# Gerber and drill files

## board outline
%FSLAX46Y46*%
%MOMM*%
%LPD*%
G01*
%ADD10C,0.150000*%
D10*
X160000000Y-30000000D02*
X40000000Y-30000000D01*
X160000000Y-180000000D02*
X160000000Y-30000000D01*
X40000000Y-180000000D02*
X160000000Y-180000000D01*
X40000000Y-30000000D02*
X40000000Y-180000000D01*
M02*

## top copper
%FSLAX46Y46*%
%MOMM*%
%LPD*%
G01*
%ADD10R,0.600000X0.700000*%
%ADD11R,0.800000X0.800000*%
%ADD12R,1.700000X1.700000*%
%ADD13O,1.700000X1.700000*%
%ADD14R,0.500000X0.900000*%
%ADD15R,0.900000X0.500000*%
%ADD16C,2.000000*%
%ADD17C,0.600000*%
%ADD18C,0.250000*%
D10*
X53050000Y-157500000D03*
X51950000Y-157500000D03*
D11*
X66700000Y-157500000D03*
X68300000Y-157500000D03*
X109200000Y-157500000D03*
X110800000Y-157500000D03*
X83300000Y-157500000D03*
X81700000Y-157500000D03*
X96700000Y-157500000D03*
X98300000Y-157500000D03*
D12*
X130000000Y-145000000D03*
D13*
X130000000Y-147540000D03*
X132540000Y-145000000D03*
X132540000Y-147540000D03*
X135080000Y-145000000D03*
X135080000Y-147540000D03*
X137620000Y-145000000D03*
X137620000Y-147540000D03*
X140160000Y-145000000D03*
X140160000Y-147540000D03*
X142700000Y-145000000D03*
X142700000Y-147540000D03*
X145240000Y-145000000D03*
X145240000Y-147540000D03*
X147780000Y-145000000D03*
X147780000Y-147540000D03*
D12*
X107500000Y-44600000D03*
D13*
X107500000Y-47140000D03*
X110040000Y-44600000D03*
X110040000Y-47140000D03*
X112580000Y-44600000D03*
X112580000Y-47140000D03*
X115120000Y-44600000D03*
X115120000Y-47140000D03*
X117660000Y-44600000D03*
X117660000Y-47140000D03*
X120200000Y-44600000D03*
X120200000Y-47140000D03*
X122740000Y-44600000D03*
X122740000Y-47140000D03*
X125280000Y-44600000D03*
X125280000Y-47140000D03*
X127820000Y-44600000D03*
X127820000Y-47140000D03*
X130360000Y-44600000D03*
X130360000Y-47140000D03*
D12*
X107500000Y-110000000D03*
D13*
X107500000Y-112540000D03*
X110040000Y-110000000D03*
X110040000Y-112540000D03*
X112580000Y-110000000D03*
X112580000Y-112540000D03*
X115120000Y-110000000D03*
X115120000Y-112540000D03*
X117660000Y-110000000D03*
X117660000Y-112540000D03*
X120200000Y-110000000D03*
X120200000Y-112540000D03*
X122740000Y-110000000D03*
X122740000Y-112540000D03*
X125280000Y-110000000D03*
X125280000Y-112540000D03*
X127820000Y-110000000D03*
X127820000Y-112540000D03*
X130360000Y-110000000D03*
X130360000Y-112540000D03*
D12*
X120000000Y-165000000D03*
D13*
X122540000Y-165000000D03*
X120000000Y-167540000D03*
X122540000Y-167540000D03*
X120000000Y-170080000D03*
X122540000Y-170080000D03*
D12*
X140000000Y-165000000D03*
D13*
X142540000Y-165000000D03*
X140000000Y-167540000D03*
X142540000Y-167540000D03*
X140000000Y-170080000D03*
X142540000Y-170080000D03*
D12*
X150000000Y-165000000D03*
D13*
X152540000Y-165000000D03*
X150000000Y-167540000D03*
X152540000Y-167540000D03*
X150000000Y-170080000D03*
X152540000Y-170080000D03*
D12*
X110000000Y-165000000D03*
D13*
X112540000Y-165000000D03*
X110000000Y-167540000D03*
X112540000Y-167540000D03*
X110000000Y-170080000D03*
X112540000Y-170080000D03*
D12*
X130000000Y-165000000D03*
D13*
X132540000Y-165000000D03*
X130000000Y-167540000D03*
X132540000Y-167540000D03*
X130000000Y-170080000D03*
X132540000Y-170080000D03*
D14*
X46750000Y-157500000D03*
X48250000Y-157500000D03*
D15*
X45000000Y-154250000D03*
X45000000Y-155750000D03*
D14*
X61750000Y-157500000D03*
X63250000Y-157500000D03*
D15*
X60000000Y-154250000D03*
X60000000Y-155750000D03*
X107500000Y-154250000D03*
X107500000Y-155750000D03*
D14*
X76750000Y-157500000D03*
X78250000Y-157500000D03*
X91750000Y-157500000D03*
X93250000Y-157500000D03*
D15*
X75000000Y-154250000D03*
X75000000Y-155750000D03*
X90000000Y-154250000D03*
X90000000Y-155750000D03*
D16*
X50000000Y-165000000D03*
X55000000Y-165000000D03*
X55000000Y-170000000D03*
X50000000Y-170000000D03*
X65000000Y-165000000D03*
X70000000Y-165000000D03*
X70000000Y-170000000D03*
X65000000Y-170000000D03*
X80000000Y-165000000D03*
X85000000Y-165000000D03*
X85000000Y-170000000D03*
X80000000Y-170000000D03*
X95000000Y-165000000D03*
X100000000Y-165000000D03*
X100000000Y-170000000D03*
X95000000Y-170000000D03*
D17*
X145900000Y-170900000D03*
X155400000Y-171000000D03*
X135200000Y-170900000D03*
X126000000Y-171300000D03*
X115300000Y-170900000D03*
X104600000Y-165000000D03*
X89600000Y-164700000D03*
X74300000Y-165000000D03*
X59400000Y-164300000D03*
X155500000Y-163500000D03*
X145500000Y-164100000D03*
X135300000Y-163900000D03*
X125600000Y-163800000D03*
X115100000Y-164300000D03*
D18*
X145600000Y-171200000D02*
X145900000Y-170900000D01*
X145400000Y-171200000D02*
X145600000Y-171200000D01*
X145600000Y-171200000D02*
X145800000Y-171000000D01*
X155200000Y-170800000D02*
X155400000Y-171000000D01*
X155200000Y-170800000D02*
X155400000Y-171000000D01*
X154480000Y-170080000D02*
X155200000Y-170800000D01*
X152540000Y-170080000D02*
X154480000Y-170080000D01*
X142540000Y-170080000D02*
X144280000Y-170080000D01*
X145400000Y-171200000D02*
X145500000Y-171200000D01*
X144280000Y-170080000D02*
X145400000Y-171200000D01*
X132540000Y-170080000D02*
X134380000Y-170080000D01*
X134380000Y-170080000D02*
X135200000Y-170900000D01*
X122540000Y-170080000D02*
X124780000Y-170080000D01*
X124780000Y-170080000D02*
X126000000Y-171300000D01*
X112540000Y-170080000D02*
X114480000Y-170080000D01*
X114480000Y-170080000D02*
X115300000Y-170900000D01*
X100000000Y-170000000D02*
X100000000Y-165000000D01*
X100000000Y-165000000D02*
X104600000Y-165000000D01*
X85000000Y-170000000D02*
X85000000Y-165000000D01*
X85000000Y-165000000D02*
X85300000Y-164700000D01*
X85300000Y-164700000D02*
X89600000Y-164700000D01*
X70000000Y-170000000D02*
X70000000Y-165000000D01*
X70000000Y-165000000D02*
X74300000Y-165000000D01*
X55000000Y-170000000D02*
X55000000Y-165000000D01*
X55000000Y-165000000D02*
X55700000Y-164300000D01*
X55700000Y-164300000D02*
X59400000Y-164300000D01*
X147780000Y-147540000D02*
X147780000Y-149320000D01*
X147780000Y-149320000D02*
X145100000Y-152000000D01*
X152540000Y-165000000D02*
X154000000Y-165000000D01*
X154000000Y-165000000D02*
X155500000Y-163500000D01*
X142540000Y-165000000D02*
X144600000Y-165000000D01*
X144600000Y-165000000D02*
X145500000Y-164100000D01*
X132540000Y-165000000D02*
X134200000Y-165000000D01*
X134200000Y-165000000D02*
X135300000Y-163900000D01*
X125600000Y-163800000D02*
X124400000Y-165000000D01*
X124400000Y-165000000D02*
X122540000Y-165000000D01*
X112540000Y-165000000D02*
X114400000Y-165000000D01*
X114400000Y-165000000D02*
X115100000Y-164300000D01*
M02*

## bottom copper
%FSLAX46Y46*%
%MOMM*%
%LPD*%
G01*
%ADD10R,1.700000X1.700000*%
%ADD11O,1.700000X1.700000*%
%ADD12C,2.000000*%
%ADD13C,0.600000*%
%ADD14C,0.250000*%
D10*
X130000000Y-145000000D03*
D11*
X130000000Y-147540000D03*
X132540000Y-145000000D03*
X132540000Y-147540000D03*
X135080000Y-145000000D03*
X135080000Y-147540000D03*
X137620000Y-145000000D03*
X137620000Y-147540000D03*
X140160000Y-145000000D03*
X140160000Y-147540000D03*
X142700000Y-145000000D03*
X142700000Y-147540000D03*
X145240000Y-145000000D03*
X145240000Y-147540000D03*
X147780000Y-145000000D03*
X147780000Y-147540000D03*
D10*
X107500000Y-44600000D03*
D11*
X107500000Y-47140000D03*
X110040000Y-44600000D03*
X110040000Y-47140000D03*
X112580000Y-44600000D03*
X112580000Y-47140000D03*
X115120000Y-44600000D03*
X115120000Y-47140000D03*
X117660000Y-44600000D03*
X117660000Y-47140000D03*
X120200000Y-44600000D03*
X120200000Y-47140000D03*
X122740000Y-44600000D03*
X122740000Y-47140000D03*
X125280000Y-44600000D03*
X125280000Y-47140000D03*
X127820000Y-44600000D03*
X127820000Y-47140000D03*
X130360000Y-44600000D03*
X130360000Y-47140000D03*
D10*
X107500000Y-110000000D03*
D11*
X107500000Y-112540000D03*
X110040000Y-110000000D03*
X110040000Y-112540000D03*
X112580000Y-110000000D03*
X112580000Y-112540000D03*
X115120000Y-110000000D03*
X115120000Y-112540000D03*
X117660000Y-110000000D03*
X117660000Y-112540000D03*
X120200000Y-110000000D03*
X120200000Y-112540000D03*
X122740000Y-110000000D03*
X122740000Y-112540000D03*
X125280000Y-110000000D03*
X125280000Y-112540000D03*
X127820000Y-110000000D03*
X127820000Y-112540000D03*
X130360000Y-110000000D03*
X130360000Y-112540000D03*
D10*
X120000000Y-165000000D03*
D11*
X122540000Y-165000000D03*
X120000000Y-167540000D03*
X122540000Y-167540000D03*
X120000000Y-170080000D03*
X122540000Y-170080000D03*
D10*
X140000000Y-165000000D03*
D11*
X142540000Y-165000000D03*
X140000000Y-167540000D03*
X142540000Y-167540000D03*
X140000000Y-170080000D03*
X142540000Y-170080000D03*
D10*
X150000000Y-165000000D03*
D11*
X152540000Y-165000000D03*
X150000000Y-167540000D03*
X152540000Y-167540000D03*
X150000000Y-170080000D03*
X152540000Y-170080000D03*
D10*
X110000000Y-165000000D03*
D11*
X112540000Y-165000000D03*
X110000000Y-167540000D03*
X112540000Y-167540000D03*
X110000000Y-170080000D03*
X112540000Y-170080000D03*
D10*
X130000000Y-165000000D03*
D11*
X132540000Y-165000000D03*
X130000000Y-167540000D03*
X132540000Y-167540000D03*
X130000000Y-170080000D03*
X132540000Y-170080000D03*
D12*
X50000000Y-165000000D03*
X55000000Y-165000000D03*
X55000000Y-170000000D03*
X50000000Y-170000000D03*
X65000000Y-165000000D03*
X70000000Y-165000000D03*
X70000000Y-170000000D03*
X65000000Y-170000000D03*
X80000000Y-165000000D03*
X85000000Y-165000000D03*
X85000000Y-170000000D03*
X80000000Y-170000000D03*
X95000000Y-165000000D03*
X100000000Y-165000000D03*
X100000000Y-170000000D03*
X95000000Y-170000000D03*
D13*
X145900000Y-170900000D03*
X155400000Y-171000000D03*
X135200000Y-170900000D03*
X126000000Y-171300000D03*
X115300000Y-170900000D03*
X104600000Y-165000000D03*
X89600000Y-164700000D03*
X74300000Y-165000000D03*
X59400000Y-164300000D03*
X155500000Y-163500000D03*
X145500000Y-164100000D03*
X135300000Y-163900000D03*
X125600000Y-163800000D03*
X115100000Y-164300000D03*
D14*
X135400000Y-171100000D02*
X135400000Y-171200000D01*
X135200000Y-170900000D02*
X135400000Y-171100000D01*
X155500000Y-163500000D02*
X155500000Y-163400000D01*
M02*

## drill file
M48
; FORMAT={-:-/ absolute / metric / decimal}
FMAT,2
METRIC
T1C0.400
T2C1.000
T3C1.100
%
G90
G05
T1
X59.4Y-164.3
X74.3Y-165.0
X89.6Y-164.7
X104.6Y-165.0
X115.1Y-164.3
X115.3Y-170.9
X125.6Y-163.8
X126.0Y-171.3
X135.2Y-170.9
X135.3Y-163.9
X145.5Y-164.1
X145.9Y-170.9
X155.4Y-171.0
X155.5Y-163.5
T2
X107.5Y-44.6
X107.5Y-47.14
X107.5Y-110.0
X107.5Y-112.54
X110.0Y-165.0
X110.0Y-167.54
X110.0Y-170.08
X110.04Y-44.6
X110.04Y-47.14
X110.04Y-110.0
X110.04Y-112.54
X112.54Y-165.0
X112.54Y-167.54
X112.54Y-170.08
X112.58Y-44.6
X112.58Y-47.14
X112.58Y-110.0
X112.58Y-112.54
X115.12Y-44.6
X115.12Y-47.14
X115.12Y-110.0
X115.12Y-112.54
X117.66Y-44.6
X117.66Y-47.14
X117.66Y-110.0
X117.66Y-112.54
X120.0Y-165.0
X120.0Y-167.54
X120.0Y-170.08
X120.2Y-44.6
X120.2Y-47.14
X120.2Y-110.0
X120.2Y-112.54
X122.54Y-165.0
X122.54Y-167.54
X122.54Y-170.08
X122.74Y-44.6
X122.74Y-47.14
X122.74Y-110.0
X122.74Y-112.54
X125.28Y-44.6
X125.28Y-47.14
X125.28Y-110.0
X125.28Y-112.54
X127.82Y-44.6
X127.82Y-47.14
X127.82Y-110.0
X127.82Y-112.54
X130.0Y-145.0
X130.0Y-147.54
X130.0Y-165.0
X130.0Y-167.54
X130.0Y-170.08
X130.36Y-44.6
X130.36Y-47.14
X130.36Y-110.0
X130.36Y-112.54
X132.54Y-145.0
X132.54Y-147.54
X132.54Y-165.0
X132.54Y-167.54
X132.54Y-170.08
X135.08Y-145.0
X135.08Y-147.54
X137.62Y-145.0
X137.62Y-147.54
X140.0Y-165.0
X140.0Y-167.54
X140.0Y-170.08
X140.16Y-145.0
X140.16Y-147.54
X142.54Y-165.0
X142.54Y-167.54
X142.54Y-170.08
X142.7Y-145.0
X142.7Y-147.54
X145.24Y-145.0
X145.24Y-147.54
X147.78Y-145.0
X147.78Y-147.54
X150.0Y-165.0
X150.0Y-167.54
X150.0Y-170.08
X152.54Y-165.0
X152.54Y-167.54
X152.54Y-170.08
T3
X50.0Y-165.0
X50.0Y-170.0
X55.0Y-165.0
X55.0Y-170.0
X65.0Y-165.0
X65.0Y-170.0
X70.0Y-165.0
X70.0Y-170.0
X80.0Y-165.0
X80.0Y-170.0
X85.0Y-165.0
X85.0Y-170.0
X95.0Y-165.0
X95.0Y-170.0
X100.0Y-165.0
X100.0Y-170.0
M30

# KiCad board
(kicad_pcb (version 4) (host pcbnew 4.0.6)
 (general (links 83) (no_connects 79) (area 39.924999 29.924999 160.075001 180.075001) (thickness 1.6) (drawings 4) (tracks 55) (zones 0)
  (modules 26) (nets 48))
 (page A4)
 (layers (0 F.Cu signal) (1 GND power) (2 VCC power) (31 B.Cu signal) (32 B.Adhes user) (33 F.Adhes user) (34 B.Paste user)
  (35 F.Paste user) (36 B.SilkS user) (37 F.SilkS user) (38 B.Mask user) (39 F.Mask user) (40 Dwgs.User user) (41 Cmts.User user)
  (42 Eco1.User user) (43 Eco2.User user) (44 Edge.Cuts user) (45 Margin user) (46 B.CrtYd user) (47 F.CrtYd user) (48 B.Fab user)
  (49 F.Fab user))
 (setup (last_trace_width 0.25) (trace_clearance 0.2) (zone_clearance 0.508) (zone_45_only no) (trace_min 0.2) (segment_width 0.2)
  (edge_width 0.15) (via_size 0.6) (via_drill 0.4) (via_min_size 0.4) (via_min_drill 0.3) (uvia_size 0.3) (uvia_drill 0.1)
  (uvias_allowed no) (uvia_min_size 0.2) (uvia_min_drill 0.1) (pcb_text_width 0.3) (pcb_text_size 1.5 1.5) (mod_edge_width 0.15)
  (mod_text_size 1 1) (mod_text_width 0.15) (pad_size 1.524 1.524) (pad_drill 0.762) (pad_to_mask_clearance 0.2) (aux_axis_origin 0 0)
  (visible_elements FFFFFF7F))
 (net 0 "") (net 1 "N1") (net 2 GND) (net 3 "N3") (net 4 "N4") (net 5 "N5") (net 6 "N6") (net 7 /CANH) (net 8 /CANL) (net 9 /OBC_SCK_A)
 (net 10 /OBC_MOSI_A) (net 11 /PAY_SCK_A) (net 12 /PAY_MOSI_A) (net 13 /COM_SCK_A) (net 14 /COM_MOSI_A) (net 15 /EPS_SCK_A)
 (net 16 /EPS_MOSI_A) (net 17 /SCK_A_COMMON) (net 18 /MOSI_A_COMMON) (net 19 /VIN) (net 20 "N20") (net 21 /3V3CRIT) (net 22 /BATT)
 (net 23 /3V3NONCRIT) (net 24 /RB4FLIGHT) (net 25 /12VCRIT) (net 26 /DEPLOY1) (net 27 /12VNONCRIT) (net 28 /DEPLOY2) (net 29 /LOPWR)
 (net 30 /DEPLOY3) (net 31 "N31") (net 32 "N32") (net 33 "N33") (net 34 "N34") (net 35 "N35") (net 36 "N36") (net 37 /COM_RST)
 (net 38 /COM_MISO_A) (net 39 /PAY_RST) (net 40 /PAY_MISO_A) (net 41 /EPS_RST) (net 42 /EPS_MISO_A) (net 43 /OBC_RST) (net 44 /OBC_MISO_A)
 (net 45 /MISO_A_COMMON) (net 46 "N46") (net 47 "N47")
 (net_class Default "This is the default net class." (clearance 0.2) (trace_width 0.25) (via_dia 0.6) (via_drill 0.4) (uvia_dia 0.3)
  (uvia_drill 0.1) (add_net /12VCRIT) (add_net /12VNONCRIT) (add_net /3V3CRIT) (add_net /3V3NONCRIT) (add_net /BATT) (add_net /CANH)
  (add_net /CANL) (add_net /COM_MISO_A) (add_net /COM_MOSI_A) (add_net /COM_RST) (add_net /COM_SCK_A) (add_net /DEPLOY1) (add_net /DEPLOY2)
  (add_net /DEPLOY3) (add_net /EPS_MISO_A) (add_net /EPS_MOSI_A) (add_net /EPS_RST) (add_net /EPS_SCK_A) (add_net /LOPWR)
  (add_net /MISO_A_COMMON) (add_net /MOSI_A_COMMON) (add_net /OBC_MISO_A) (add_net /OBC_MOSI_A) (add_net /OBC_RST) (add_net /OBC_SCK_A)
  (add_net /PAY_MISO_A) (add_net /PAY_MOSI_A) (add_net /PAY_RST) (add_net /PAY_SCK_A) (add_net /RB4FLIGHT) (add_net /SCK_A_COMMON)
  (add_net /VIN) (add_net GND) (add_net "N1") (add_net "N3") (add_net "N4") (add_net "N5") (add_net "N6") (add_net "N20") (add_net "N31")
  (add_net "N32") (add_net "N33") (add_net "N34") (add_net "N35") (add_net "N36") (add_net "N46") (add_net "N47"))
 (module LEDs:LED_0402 (layer F.Cu) (at 52.5 157.5)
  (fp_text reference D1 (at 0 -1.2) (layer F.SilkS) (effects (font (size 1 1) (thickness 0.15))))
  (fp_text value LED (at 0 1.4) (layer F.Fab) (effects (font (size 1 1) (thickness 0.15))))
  (pad 2 smd rect (at 0.55 0 180) (size 0.6 0.7) (layers F.Cu F.Paste F.Mask) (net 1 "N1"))
  (pad 1 smd rect (at -0.55 0 180) (size 0.6 0.7) (layers F.Cu F.Paste F.Mask) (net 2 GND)))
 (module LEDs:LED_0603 (layer F.Cu) (at 67.5 157.5 180)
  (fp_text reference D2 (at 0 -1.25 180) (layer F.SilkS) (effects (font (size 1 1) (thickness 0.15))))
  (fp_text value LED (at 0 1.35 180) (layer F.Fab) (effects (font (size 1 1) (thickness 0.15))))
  (pad 2 smd rect (at 0.8 0) (size 0.8 0.8) (layers F.Cu F.Paste F.Mask) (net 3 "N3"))
  (pad 1 smd rect (at -0.8 0) (size 0.8 0.8) (layers F.Cu F.Paste F.Mask) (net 2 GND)))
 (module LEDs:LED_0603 (layer F.Cu) (at 110 157.5 180)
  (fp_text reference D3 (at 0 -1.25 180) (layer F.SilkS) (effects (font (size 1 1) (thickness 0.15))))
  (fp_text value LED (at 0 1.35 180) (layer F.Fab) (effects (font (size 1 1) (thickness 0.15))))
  (pad 2 smd rect (at 0.8 0) (size 0.8 0.8) (layers F.Cu F.Paste F.Mask) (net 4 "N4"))
  (pad 1 smd rect (at -0.8 0) (size 0.8 0.8) (layers F.Cu F.Paste F.Mask) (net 2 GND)))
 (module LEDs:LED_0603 (layer F.Cu) (at 82.5 157.5)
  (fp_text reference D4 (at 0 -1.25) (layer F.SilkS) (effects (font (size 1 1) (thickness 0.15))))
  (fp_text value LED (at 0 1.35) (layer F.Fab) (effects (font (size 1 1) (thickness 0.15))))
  (pad 2 smd rect (at 0.8 0 180) (size 0.8 0.8) (layers F.Cu F.Paste F.Mask) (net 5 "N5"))
  (pad 1 smd rect (at -0.8 0 180) (size 0.8 0.8) (layers F.Cu F.Paste F.Mask) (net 2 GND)))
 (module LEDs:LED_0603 (layer F.Cu) (at 97.5 157.5 180)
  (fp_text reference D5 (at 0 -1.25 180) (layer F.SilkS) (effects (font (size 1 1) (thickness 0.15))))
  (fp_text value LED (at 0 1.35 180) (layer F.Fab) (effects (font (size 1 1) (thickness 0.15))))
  (pad 2 smd rect (at 0.8 0) (size 0.8 0.8) (layers F.Cu F.Paste F.Mask) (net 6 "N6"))
  (pad 1 smd rect (at -0.8 0) (size 0.8 0.8) (layers F.Cu F.Paste F.Mask) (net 2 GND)))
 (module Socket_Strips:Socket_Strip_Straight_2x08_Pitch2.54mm (layer F.Cu) (at 130 145 90)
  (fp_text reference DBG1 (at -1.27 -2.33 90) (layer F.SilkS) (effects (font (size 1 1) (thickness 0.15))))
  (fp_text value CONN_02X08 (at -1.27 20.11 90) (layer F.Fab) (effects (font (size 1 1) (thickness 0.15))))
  (pad 1 thru_hole rect (at 0 0 90) (size 1.7 1.7) (drill 1) (layers *.Cu *.Mask) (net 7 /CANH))
  (pad 2 thru_hole oval (at -2.54 0 90) (size 1.7 1.7) (drill 1) (layers *.Cu *.Mask) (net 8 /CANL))
  (pad 3 thru_hole oval (at 0 2.54 90) (size 1.7 1.7) (drill 1) (layers *.Cu *.Mask) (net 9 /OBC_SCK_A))
  (pad 4 thru_hole oval (at -2.54 2.54 90) (size 1.7 1.7) (drill 1) (layers *.Cu *.Mask) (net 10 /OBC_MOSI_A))
  (pad 5 thru_hole oval (at 0 5.08 90) (size 1.7 1.7) (drill 1) (layers *.Cu *.Mask) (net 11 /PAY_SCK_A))
  (pad 6 thru_hole oval (at -2.54 5.08 90) (size 1.7 1.7) (drill 1) (layers *.Cu *.Mask) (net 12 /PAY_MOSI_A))
  (pad 7 thru_hole oval (at 0 7.62 90) (size 1.7 1.7) (drill 1) (layers *.Cu *.Mask) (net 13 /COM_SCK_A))
  (pad 8 thru_hole oval (at -2.54 7.62 90) (size 1.7 1.7) (drill 1) (layers *.Cu *.Mask) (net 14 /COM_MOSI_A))
  (pad 9 thru_hole oval (at 0 10.16 90) (size 1.7 1.7) (drill 1) (layers *.Cu *.Mask) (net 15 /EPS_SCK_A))
  (pad 10 thru_hole oval (at -2.54 10.16 90) (size 1.7 1.7) (drill 1) (layers *.Cu *.Mask) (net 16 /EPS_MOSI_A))
  (pad 11 thru_hole oval (at 0 12.7 90) (size 1.7 1.7) (drill 1) (layers *.Cu *.Mask) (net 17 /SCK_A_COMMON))
  (pad 12 thru_hole oval (at -2.54 12.7 90) (size 1.7 1.7) (drill 1) (layers *.Cu *.Mask) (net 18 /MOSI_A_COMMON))
  (pad 13 thru_hole oval (at 0 15.24 90) (size 1.7 1.7) (drill 1) (layers *.Cu *.Mask) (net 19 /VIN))
  (pad 14 thru_hole oval (at -2.54 15.24 90) (size 1.7 1.7) (drill 1) (layers *.Cu *.Mask) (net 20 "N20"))
  (pad 15 thru_hole oval (at 0 17.78 90) (size 1.7 1.7) (drill 1) (layers *.Cu *.Mask) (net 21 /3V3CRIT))
  (pad 16 thru_hole oval (at -2.54 17.78 90) (size 1.7 1.7) (drill 1) (layers *.Cu *.Mask) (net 2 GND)))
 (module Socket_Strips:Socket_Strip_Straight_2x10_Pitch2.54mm (layer F.Cu) (at 107.5 44.6 90)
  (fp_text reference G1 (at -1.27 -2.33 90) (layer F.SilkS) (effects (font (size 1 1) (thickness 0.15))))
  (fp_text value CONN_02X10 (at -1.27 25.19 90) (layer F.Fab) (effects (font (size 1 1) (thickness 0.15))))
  (pad 1 thru_hole rect (at 0 0 90) (size 1.7 1.7) (drill 1) (layers *.Cu *.Mask) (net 21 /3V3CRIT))
  (pad 2 thru_hole oval (at -2.54 0 90) (size 1.7 1.7) (drill 1) (layers *.Cu *.Mask) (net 19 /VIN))
  (pad 3 thru_hole oval (at 0 2.54 90) (size 1.7 1.7) (drill 1) (layers *.Cu *.Mask) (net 2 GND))
  (pad 4 thru_hole oval (at -2.54 2.54 90) (size 1.7 1.7) (drill 1) (layers *.Cu *.Mask) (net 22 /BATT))
  (pad 5 thru_hole oval (at 0 5.08 90) (size 1.7 1.7) (drill 1) (layers *.Cu *.Mask) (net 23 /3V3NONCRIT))
  (pad 6 thru_hole oval (at -2.54 5.08 90) (size 1.7 1.7) (drill 1) (layers *.Cu *.Mask) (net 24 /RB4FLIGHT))
  (pad 7 thru_hole oval (at 0 7.62 90) (size 1.7 1.7) (drill 1) (layers *.Cu *.Mask) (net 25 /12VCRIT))
  (pad 8 thru_hole oval (at -2.54 7.62 90) (size 1.7 1.7) (drill 1) (layers *.Cu *.Mask) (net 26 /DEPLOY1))
  (pad 9 thru_hole oval (at 0 10.16 90) (size 1.7 1.7) (drill 1) (layers *.Cu *.Mask) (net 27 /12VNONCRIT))
  (pad 10 thru_hole oval (at -2.54 10.16 90) (size 1.7 1.7) (drill 1) (layers *.Cu *.Mask) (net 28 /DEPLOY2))
  (pad 11 thru_hole oval (at 0 12.7 90) (size 1.7 1.7) (drill 1) (layers *.Cu *.Mask) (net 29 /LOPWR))
  (pad 12 thru_hole oval (at -2.54 12.7 90) (size 1.7 1.7) (drill 1) (layers *.Cu *.Mask) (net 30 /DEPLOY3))
  (pad 13 thru_hole oval (at 0 15.24 90) (size 1.7 1.7) (drill 1) (layers *.Cu *.Mask) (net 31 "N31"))
  (pad 14 thru_hole oval (at -2.54 15.24 90) (size 1.7 1.7) (drill 1) (layers *.Cu *.Mask) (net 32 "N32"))
  (pad 15 thru_hole oval (at 0 17.78 90) (size 1.7 1.7) (drill 1) (layers *.Cu *.Mask) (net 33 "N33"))
  (pad 16 thru_hole oval (at -2.54 17.78 90) (size 1.7 1.7) (drill 1) (layers *.Cu *.Mask) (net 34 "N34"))
  (pad 17 thru_hole oval (at 0 20.32 90) (size 1.7 1.7) (drill 1) (layers *.Cu *.Mask) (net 7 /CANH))
  (pad 18 thru_hole oval (at -2.54 20.32 90) (size 1.7 1.7) (drill 1) (layers *.Cu *.Mask) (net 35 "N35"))
  (pad 19 thru_hole oval (at 0 22.86 90) (size 1.7 1.7) (drill 1) (layers *.Cu *.Mask) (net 8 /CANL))
  (pad 20 thru_hole oval (at -2.54 22.86 90) (size 1.7 1.7) (drill 1) (layers *.Cu *.Mask) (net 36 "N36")))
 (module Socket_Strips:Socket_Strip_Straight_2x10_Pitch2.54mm (layer F.Cu) (at 107.5 110 90)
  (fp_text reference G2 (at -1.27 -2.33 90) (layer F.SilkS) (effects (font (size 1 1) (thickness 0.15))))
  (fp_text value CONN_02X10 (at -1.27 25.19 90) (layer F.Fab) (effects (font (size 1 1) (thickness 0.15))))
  (pad 1 thru_hole rect (at 0 0 90) (size 1.7 1.7) (drill 1) (layers *.Cu *.Mask) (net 14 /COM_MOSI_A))
  (pad 2 thru_hole oval (at -2.54 0 90) (size 1.7 1.7) (drill 1) (layers *.Cu *.Mask) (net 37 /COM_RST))
  (pad 3 thru_hole oval (at 0 2.54 90) (size 1.7 1.7) (drill 1) (layers *.Cu *.Mask) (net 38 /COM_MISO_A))
  (pad 4 thru_hole oval (at -2.54 2.54 90) (size 1.7 1.7) (drill 1) (layers *.Cu *.Mask) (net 13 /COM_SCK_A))
  (pad 5 thru_hole oval (at 0 5.08 90) (size 1.7 1.7) (drill 1) (layers *.Cu *.Mask) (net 12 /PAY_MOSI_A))
  (pad 6 thru_hole oval (at -2.54 5.08 90) (size 1.7 1.7) (drill 1) (layers *.Cu *.Mask) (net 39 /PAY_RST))
  (pad 7 thru_hole oval (at 0 7.62 90) (size 1.7 1.7) (drill 1) (layers *.Cu *.Mask) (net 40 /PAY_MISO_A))
  (pad 8 thru_hole oval (at -2.54 7.62 90) (size 1.7 1.7) (drill 1) (layers *.Cu *.Mask) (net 11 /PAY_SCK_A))
  (pad 9 thru_hole oval (at 0 10.16 90) (size 1.7 1.7) (drill 1) (layers *.Cu *.Mask) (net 16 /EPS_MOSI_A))
  (pad 10 thru_hole oval (at -2.54 10.16 90) (size 1.7 1.7) (drill 1) (layers *.Cu *.Mask) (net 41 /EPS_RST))
  (pad 11 thru_hole oval (at 0 12.7 90) (size 1.7 1.7) (drill 1) (layers *.Cu *.Mask) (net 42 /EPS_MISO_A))
  (pad 12 thru_hole oval (at -2.54 12.7 90) (size 1.7 1.7) (drill 1) (layers *.Cu *.Mask) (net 15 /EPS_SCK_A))
  (pad 13 thru_hole oval (at 0 15.24 90) (size 1.7 1.7) (drill 1) (layers *.Cu *.Mask) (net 10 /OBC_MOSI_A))
  (pad 14 thru_hole oval (at -2.54 15.24 90) (size 1.7 1.7) (drill 1) (layers *.Cu *.Mask) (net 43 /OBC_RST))
  (pad 15 thru_hole oval (at 0 17.78 90) (size 1.7 1.7) (drill 1) (layers *.Cu *.Mask) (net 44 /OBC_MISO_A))
  (pad 16 thru_hole oval (at -2.54 17.78 90) (size 1.7 1.7) (drill 1) (layers *.Cu *.Mask) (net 9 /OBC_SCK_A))
  (pad 17 thru_hole oval (at 0 20.32 90) (size 1.7 1.7) (drill 1) (layers *.Cu *.Mask) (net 18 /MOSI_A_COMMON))
  (pad 18 thru_hole oval (at -2.54 20.32 90) (size 1.7 1.7) (drill 1) (layers *.Cu *.Mask) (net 17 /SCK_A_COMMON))
  (pad 19 thru_hole oval (at 0 22.86 90) (size 1.7 1.7) (drill 1) (layers *.Cu *.Mask) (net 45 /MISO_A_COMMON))
  (pad 20 thru_hole oval (at -2.54 22.86 90) (size 1.7 1.7) (drill 1) (layers *.Cu *.Mask) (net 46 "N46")))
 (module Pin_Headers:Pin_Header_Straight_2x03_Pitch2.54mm (layer F.Cu) (at 120 165)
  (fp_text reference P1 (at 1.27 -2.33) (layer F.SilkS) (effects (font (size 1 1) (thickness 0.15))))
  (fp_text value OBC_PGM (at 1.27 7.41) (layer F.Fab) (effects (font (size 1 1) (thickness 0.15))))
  (pad 1 thru_hole rect (at 0 0) (size 1.7 1.7) (drill 1) (layers *.Cu *.Mask) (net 44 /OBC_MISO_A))
  (pad 2 thru_hole oval (at 2.54 0) (size 1.7 1.7) (drill 1) (layers *.Cu *.Mask) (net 21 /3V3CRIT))
  (pad 3 thru_hole oval (at 0 2.54) (size 1.7 1.7) (drill 1) (layers *.Cu *.Mask) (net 9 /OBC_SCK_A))
  (pad 4 thru_hole oval (at 2.54 2.54) (size 1.7 1.7) (drill 1) (layers *.Cu *.Mask) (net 10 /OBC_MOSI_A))
  (pad 5 thru_hole oval (at 0 5.08) (size 1.7 1.7) (drill 1) (layers *.Cu *.Mask) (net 43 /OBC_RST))
  (pad 6 thru_hole oval (at 2.54 5.08) (size 1.7 1.7) (drill 1) (layers *.Cu *.Mask) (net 2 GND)))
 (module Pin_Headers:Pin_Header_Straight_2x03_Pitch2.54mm (layer F.Cu) (at 140 165)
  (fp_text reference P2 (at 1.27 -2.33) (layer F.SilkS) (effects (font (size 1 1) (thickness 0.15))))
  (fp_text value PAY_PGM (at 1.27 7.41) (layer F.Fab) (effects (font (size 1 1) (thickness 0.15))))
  (pad 1 thru_hole rect (at 0 0) (size 1.7 1.7) (drill 1) (layers *.Cu *.Mask) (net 40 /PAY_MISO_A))
  (pad 2 thru_hole oval (at 2.54 0) (size 1.7 1.7) (drill 1) (layers *.Cu *.Mask) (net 21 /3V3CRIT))
  (pad 3 thru_hole oval (at 0 2.54) (size 1.7 1.7) (drill 1) (layers *.Cu *.Mask) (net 11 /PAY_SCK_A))
  (pad 4 thru_hole oval (at 2.54 2.54) (size 1.7 1.7) (drill 1) (layers *.Cu *.Mask) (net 12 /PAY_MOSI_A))
  (pad 5 thru_hole oval (at 0 5.08) (size 1.7 1.7) (drill 1) (layers *.Cu *.Mask) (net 39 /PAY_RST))
  (pad 6 thru_hole oval (at 2.54 5.08) (size 1.7 1.7) (drill 1) (layers *.Cu *.Mask) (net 2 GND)))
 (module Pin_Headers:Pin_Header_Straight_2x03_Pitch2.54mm (layer F.Cu) (at 150 165)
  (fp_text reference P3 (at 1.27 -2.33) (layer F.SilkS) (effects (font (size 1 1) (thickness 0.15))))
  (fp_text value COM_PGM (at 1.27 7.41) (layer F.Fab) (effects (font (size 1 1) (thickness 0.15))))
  (pad 1 thru_hole rect (at 0 0) (size 1.7 1.7) (drill 1) (layers *.Cu *.Mask) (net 38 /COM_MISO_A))
  (pad 2 thru_hole oval (at 2.54 0) (size 1.7 1.7) (drill 1) (layers *.Cu *.Mask) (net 21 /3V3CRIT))
  (pad 3 thru_hole oval (at 0 2.54) (size 1.7 1.7) (drill 1) (layers *.Cu *.Mask) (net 13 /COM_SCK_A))
  (pad 4 thru_hole oval (at 2.54 2.54) (size 1.7 1.7) (drill 1) (layers *.Cu *.Mask) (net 14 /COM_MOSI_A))
  (pad 5 thru_hole oval (at 0 5.08) (size 1.7 1.7) (drill 1) (layers *.Cu *.Mask) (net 37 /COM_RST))
  (pad 6 thru_hole oval (at 2.54 5.08) (size 1.7 1.7) (drill 1) (layers *.Cu *.Mask) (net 2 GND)))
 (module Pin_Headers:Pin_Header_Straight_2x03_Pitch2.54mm (layer F.Cu) (at 110 165)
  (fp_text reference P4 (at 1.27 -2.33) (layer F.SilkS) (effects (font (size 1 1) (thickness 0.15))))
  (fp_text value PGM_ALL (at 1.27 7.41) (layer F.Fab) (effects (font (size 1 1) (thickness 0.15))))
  (pad 1 thru_hole rect (at 0 0) (size 1.7 1.7) (drill 1) (layers *.Cu *.Mask) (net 45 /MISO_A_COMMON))
  (pad 2 thru_hole oval (at 2.54 0) (size 1.7 1.7) (drill 1) (layers *.Cu *.Mask) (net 21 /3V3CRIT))
  (pad 3 thru_hole oval (at 0 2.54) (size 1.7 1.7) (drill 1) (layers *.Cu *.Mask) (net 17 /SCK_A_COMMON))
  (pad 4 thru_hole oval (at 2.54 2.54) (size 1.7 1.7) (drill 1) (layers *.Cu *.Mask) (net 18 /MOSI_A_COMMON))
  (pad 5 thru_hole oval (at 0 5.08) (size 1.7 1.7) (drill 1) (layers *.Cu *.Mask) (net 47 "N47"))
  (pad 6 thru_hole oval (at 2.54 5.08) (size 1.7 1.7) (drill 1) (layers *.Cu *.Mask) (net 2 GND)))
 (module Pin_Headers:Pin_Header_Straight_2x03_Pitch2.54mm (layer F.Cu) (at 130 165)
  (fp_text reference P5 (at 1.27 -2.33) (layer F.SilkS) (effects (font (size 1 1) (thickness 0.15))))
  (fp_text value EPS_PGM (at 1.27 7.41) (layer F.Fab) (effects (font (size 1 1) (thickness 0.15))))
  (pad 1 thru_hole rect (at 0 0) (size 1.7 1.7) (drill 1) (layers *.Cu *.Mask) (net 42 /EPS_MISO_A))
  (pad 2 thru_hole oval (at 2.54 0) (size 1.7 1.7) (drill 1) (layers *.Cu *.Mask) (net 21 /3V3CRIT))
  (pad 3 thru_hole oval (at 0 2.54) (size 1.7 1.7) (drill 1) (layers *.Cu *.Mask) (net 15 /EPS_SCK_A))
  (pad 4 thru_hole oval (at 2.54 2.54) (size 1.7 1.7) (drill 1) (layers *.Cu *.Mask) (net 16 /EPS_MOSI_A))
  (pad 5 thru_hole oval (at 0 5.08) (size 1.7 1.7) (drill 1) (layers *.Cu *.Mask) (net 41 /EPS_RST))
  (pad 6 thru_hole oval (at 2.54 5.08) (size 1.7 1.7) (drill 1) (layers *.Cu *.Mask) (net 2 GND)))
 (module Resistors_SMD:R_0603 (layer F.Cu) (at 47.5 157.5)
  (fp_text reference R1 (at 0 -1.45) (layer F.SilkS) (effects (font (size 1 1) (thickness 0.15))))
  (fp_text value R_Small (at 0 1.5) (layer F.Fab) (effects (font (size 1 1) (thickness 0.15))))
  (pad 1 smd rect (at -0.75 0) (size 0.5 0.9) (layers F.Cu F.Paste F.Mask) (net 43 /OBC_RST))
  (pad 2 smd rect (at 0.75 0) (size 0.5 0.9) (layers F.Cu F.Paste F.Mask) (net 1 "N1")))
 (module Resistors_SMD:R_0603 (layer F.Cu) (at 45 155 270)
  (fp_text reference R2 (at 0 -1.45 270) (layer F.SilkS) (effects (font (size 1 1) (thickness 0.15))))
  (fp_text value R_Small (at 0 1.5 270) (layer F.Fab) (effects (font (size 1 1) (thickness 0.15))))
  (pad 1 smd rect (at -0.75 0 270) (size 0.5 0.9) (layers F.Cu F.Paste F.Mask) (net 21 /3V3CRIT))
  (pad 2 smd rect (at 0.75 0 270) (size 0.5 0.9) (layers F.Cu F.Paste F.Mask) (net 43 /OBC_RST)))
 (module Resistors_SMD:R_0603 (layer F.Cu) (at 62.5 157.5)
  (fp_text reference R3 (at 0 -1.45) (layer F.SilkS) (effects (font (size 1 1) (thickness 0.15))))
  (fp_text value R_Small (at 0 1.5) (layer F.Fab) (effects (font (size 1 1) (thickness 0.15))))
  (pad 1 smd rect (at -0.75 0) (size 0.5 0.9) (layers F.Cu F.Paste F.Mask) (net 39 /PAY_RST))
  (pad 2 smd rect (at 0.75 0) (size 0.5 0.9) (layers F.Cu F.Paste F.Mask) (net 3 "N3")))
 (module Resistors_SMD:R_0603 (layer F.Cu) (at 60 155 270)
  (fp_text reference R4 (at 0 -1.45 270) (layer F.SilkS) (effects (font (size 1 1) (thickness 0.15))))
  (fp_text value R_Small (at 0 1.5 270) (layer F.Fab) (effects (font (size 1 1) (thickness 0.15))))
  (pad 1 smd rect (at -0.75 0 270) (size 0.5 0.9) (layers F.Cu F.Paste F.Mask) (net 21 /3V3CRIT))
  (pad 2 smd rect (at 0.75 0 270) (size 0.5 0.9) (layers F.Cu F.Paste F.Mask) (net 39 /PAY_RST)))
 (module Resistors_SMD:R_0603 (layer F.Cu) (at 107.5 155 270)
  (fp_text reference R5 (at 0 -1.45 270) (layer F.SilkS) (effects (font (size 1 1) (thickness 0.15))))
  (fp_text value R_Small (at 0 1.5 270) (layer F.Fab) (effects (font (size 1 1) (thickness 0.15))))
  (pad 1 smd rect (at -0.75 0 270) (size 0.5 0.9) (layers F.Cu F.Paste F.Mask) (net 21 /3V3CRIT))
  (pad 2 smd rect (at 0.75 0 270) (size 0.5 0.9) (layers F.Cu F.Paste F.Mask) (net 4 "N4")))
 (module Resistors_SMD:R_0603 (layer F.Cu) (at 77.5 157.5)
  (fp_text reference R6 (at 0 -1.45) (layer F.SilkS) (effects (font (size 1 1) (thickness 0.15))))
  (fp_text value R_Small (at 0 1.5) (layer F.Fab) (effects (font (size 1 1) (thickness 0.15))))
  (pad 1 smd rect (at -0.75 0) (size 0.5 0.9) (layers F.Cu F.Paste F.Mask) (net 37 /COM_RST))
  (pad 2 smd rect (at 0.75 0) (size 0.5 0.9) (layers F.Cu F.Paste F.Mask) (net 5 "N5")))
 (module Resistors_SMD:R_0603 (layer F.Cu) (at 92.5 157.5)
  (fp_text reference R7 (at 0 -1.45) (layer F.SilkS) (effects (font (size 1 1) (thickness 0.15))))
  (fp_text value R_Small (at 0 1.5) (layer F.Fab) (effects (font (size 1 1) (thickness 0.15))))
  (pad 1 smd rect (at -0.75 0) (size 0.5 0.9) (layers F.Cu F.Paste F.Mask) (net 41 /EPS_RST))
  (pad 2 smd rect (at 0.75 0) (size 0.5 0.9) (layers F.Cu F.Paste F.Mask) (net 6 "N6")))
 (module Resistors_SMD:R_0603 (layer F.Cu) (at 75 155 270)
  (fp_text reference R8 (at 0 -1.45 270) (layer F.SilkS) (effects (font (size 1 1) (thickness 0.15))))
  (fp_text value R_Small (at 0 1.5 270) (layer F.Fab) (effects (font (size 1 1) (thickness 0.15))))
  (pad 1 smd rect (at -0.75 0 270) (size 0.5 0.9) (layers F.Cu F.Paste F.Mask) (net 21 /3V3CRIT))
  (pad 2 smd rect (at 0.75 0 270) (size 0.5 0.9) (layers F.Cu F.Paste F.Mask) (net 37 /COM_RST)))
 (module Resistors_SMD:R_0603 (layer F.Cu) (at 90 155 270)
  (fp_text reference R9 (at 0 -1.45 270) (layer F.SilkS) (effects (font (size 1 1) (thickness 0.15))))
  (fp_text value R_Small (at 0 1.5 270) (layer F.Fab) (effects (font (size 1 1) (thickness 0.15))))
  (pad 1 smd rect (at -0.75 0 270) (size 0.5 0.9) (layers F.Cu F.Paste F.Mask) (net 21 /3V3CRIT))
  (pad 2 smd rect (at 0.75 0 270) (size 0.5 0.9) (layers F.Cu F.Paste F.Mask) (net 41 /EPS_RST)))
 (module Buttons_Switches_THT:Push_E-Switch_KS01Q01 (layer F.Cu) (at 50 165)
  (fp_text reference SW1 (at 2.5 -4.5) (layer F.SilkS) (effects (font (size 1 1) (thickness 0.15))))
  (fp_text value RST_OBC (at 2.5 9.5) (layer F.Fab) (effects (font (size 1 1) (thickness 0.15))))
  (pad 1 thru_hole circle (at 0 0) (size 2 2) (drill 1.1) (layers *.Cu *.Mask) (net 43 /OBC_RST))
  (pad 2 thru_hole circle (at 5 0) (size 2 2) (drill 1.1) (layers *.Cu *.Mask) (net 2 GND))
  (pad 4 thru_hole circle (at 5 5) (size 2 2) (drill 1.1) (layers *.Cu *.Mask) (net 2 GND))
  (pad 3 thru_hole circle (at 0 5) (size 2 2) (drill 1.1) (layers *.Cu *.Mask) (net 43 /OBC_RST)))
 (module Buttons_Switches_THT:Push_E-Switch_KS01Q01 (layer F.Cu) (at 65 165)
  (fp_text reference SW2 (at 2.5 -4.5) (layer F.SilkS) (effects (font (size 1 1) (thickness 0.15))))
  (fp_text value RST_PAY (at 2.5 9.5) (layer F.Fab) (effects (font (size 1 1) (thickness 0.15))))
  (pad 1 thru_hole circle (at 0 0) (size 2 2) (drill 1.1) (layers *.Cu *.Mask) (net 39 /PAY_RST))
  (pad 2 thru_hole circle (at 5 0) (size 2 2) (drill 1.1) (layers *.Cu *.Mask) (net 2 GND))
  (pad 4 thru_hole circle (at 5 5) (size 2 2) (drill 1.1) (layers *.Cu *.Mask) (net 2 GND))
  (pad 3 thru_hole circle (at 0 5) (size 2 2) (drill 1.1) (layers *.Cu *.Mask) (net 39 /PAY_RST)))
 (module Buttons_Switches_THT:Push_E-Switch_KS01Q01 (layer F.Cu) (at 80 165)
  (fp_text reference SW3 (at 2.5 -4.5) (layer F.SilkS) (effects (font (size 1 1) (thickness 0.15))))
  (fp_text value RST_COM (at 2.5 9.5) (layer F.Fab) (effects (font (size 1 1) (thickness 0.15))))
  (pad 1 thru_hole circle (at 0 0) (size 2 2) (drill 1.1) (layers *.Cu *.Mask) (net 37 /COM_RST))
  (pad 2 thru_hole circle (at 5 0) (size 2 2) (drill 1.1) (layers *.Cu *.Mask) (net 2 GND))
  (pad 4 thru_hole circle (at 5 5) (size 2 2) (drill 1.1) (layers *.Cu *.Mask) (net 2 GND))
  (pad 3 thru_hole circle (at 0 5) (size 2 2) (drill 1.1) (layers *.Cu *.Mask) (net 37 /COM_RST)))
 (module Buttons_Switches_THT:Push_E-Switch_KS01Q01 (layer F.Cu) (at 95 165)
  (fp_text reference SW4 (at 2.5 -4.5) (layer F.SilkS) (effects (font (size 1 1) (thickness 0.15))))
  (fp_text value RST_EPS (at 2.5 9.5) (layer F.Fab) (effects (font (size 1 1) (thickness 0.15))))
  (pad 1 thru_hole circle (at 0 0) (size 2 2) (drill 1.1) (layers *.Cu *.Mask) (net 41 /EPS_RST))
  (pad 2 thru_hole circle (at 5 0) (size 2 2) (drill 1.1) (layers *.Cu *.Mask) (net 2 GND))
  (pad 4 thru_hole circle (at 5 5) (size 2 2) (drill 1.1) (layers *.Cu *.Mask) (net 2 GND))
  (pad 3 thru_hole circle (at 0 5) (size 2 2) (drill 1.1) (layers *.Cu *.Mask) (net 41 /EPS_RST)))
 (gr_line (start 160 30) (end 40 30) (angle 90) (layer Edge.Cuts) (width 0.15))
 (gr_line (start 160 180) (end 160 30) (angle 90) (layer Edge.Cuts) (width 0.15))
 (gr_line (start 40 180) (end 160 180) (angle 90) (layer Edge.Cuts) (width 0.15))
 (gr_line (start 40 30) (end 40 180) (angle 90) (layer Edge.Cuts) (width 0.15))
 (segment (start 145.6 171.2) (end 145.9 170.9) (width 0.25) (layer F.Cu) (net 2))
 (via (at 145.9 170.9) (size 0.6) (drill 0.4) (layers F.Cu B.Cu) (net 2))
 (segment (start 145.4 171.2) (end 145.6 171.2) (width 0.25) (layer F.Cu) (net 2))
 (segment (start 145.6 171.2) (end 145.8 171) (width 0.25) (layer F.Cu) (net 2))
 (segment (start 155.2 170.8) (end 155.4 171) (width 0.25) (layer F.Cu) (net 2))
 (segment (start 155.2 170.8) (end 155.4 171) (width 0.25) (layer F.Cu) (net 2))
 (segment (start 154.48 170.08) (end 155.2 170.8) (width 0.25) (layer F.Cu) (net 2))
 (segment (start 152.54 170.08) (end 154.48 170.08) (width 0.25) (layer F.Cu) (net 2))
 (via (at 155.4 171) (size 0.6) (drill 0.4) (layers F.Cu B.Cu) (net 2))
 (segment (start 142.54 170.08) (end 144.28 170.08) (width 0.25) (layer F.Cu) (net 2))
 (segment (start 145.4 171.2) (end 145.5 171.2) (width 0.25) (layer F.Cu) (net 2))
 (segment (start 144.28 170.08) (end 145.4 171.2) (width 0.25) (layer F.Cu) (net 2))
 (segment (start 132.54 170.08) (end 134.38 170.08) (width 0.25) (layer F.Cu) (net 2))
 (segment (start 135.4 171.1) (end 135.4 171.2) (width 0.25) (layer B.Cu) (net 2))
 (segment (start 135.2 170.9) (end 135.4 171.1) (width 0.25) (layer B.Cu) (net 2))
 (via (at 135.2 170.9) (size 0.6) (drill 0.4) (layers F.Cu B.Cu) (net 2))
 (segment (start 134.38 170.08) (end 135.2 170.9) (width 0.25) (layer F.Cu) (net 2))
 (segment (start 122.54 170.08) (end 124.78 170.08) (width 0.25) (layer F.Cu) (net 2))
 (via (at 126 171.3) (size 0.6) (drill 0.4) (layers F.Cu B.Cu) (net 2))
 (segment (start 124.78 170.08) (end 126 171.3) (width 0.25) (layer F.Cu) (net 2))
 (segment (start 112.54 170.08) (end 114.48 170.08) (width 0.25) (layer F.Cu) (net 2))
 (via (at 115.3 170.9) (size 0.6) (drill 0.4) (layers F.Cu B.Cu) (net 2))
 (segment (start 114.48 170.08) (end 115.3 170.9) (width 0.25) (layer F.Cu) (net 2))
 (segment (start 100 170) (end 100 165) (width 0.25) (layer F.Cu) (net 2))
 (segment (start 100 165) (end 104.6 165) (width 0.25) (layer F.Cu) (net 2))
 (via (at 104.6 165) (size 0.6) (drill 0.4) (layers F.Cu B.Cu) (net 2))
 (segment (start 85 170) (end 85 165) (width 0.25) (layer F.Cu) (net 2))
 (segment (start 85 165) (end 85.3 164.7) (width 0.25) (layer F.Cu) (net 2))
 (segment (start 85.3 164.7) (end 89.6 164.7) (width 0.25) (layer F.Cu) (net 2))
 (via (at 89.6 164.7) (size 0.6) (drill 0.4) (layers F.Cu B.Cu) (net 2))
 (segment (start 70 170) (end 70 165) (width 0.25) (layer F.Cu) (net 2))
 (segment (start 70 165) (end 74.3 165) (width 0.25) (layer F.Cu) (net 2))
 (via (at 74.3 165) (size 0.6) (drill 0.4) (layers F.Cu B.Cu) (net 2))
 (segment (start 55 170) (end 55 165) (width 0.25) (layer F.Cu) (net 2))
 (segment (start 55 165) (end 55.7 164.3) (width 0.25) (layer F.Cu) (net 2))
 (segment (start 55.7 164.3) (end 59.4 164.3) (width 0.25) (layer F.Cu) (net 2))
 (via (at 59.4 164.3) (size 0.6) (drill 0.4) (layers F.Cu B.Cu) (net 2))
 (segment (start 147.78 147.54) (end 147.78 149.32) (width 0.25) (layer F.Cu) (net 2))
 (segment (start 147.78 149.32) (end 145.1 152) (width 0.25) (layer F.Cu) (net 2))
 (segment (start 152.54 165) (end 154 165) (width 0.25) (layer F.Cu) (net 21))
 (segment (start 155.5 163.5) (end 155.5 163.4) (width 0.25) (layer B.Cu) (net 21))
 (via (at 155.5 163.5) (size 0.6) (drill 0.4) (layers F.Cu B.Cu) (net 21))
 (segment (start 154 165) (end 155.5 163.5) (width 0.25) (layer F.Cu) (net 21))
 (segment (start 142.54 165) (end 144.6 165) (width 0.25) (layer F.Cu) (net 21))
 (via (at 145.5 164.1) (size 0.6) (drill 0.4) (layers F.Cu B.Cu) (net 21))
 (segment (start 144.6 165) (end 145.5 164.1) (width 0.25) (layer F.Cu) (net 21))
 (segment (start 132.54 165) (end 134.2 165) (width 0.25) (layer F.Cu) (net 21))
 (via (at 135.3 163.9) (size 0.6) (drill 0.4) (layers F.Cu B.Cu) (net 21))
 (segment (start 134.2 165) (end 135.3 163.9) (width 0.25) (layer F.Cu) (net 21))
 (via (at 125.6 163.8) (size 0.6) (drill 0.4) (layers F.Cu B.Cu) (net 21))
 (segment (start 125.6 163.8) (end 124.4 165) (width 0.25) (layer F.Cu) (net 21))
 (segment (start 124.4 165) (end 122.54 165) (width 0.25) (layer F.Cu) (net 21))
 (segment (start 112.54 165) (end 114.4 165) (width 0.25) (layer F.Cu) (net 21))
 (via (at 115.1 164.3) (size 0.6) (drill 0.4) (layers F.Cu B.Cu) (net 21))
 (segment (start 114.4 165) (end 115.1 164.3) (width 0.25) (layer F.Cu) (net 21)))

